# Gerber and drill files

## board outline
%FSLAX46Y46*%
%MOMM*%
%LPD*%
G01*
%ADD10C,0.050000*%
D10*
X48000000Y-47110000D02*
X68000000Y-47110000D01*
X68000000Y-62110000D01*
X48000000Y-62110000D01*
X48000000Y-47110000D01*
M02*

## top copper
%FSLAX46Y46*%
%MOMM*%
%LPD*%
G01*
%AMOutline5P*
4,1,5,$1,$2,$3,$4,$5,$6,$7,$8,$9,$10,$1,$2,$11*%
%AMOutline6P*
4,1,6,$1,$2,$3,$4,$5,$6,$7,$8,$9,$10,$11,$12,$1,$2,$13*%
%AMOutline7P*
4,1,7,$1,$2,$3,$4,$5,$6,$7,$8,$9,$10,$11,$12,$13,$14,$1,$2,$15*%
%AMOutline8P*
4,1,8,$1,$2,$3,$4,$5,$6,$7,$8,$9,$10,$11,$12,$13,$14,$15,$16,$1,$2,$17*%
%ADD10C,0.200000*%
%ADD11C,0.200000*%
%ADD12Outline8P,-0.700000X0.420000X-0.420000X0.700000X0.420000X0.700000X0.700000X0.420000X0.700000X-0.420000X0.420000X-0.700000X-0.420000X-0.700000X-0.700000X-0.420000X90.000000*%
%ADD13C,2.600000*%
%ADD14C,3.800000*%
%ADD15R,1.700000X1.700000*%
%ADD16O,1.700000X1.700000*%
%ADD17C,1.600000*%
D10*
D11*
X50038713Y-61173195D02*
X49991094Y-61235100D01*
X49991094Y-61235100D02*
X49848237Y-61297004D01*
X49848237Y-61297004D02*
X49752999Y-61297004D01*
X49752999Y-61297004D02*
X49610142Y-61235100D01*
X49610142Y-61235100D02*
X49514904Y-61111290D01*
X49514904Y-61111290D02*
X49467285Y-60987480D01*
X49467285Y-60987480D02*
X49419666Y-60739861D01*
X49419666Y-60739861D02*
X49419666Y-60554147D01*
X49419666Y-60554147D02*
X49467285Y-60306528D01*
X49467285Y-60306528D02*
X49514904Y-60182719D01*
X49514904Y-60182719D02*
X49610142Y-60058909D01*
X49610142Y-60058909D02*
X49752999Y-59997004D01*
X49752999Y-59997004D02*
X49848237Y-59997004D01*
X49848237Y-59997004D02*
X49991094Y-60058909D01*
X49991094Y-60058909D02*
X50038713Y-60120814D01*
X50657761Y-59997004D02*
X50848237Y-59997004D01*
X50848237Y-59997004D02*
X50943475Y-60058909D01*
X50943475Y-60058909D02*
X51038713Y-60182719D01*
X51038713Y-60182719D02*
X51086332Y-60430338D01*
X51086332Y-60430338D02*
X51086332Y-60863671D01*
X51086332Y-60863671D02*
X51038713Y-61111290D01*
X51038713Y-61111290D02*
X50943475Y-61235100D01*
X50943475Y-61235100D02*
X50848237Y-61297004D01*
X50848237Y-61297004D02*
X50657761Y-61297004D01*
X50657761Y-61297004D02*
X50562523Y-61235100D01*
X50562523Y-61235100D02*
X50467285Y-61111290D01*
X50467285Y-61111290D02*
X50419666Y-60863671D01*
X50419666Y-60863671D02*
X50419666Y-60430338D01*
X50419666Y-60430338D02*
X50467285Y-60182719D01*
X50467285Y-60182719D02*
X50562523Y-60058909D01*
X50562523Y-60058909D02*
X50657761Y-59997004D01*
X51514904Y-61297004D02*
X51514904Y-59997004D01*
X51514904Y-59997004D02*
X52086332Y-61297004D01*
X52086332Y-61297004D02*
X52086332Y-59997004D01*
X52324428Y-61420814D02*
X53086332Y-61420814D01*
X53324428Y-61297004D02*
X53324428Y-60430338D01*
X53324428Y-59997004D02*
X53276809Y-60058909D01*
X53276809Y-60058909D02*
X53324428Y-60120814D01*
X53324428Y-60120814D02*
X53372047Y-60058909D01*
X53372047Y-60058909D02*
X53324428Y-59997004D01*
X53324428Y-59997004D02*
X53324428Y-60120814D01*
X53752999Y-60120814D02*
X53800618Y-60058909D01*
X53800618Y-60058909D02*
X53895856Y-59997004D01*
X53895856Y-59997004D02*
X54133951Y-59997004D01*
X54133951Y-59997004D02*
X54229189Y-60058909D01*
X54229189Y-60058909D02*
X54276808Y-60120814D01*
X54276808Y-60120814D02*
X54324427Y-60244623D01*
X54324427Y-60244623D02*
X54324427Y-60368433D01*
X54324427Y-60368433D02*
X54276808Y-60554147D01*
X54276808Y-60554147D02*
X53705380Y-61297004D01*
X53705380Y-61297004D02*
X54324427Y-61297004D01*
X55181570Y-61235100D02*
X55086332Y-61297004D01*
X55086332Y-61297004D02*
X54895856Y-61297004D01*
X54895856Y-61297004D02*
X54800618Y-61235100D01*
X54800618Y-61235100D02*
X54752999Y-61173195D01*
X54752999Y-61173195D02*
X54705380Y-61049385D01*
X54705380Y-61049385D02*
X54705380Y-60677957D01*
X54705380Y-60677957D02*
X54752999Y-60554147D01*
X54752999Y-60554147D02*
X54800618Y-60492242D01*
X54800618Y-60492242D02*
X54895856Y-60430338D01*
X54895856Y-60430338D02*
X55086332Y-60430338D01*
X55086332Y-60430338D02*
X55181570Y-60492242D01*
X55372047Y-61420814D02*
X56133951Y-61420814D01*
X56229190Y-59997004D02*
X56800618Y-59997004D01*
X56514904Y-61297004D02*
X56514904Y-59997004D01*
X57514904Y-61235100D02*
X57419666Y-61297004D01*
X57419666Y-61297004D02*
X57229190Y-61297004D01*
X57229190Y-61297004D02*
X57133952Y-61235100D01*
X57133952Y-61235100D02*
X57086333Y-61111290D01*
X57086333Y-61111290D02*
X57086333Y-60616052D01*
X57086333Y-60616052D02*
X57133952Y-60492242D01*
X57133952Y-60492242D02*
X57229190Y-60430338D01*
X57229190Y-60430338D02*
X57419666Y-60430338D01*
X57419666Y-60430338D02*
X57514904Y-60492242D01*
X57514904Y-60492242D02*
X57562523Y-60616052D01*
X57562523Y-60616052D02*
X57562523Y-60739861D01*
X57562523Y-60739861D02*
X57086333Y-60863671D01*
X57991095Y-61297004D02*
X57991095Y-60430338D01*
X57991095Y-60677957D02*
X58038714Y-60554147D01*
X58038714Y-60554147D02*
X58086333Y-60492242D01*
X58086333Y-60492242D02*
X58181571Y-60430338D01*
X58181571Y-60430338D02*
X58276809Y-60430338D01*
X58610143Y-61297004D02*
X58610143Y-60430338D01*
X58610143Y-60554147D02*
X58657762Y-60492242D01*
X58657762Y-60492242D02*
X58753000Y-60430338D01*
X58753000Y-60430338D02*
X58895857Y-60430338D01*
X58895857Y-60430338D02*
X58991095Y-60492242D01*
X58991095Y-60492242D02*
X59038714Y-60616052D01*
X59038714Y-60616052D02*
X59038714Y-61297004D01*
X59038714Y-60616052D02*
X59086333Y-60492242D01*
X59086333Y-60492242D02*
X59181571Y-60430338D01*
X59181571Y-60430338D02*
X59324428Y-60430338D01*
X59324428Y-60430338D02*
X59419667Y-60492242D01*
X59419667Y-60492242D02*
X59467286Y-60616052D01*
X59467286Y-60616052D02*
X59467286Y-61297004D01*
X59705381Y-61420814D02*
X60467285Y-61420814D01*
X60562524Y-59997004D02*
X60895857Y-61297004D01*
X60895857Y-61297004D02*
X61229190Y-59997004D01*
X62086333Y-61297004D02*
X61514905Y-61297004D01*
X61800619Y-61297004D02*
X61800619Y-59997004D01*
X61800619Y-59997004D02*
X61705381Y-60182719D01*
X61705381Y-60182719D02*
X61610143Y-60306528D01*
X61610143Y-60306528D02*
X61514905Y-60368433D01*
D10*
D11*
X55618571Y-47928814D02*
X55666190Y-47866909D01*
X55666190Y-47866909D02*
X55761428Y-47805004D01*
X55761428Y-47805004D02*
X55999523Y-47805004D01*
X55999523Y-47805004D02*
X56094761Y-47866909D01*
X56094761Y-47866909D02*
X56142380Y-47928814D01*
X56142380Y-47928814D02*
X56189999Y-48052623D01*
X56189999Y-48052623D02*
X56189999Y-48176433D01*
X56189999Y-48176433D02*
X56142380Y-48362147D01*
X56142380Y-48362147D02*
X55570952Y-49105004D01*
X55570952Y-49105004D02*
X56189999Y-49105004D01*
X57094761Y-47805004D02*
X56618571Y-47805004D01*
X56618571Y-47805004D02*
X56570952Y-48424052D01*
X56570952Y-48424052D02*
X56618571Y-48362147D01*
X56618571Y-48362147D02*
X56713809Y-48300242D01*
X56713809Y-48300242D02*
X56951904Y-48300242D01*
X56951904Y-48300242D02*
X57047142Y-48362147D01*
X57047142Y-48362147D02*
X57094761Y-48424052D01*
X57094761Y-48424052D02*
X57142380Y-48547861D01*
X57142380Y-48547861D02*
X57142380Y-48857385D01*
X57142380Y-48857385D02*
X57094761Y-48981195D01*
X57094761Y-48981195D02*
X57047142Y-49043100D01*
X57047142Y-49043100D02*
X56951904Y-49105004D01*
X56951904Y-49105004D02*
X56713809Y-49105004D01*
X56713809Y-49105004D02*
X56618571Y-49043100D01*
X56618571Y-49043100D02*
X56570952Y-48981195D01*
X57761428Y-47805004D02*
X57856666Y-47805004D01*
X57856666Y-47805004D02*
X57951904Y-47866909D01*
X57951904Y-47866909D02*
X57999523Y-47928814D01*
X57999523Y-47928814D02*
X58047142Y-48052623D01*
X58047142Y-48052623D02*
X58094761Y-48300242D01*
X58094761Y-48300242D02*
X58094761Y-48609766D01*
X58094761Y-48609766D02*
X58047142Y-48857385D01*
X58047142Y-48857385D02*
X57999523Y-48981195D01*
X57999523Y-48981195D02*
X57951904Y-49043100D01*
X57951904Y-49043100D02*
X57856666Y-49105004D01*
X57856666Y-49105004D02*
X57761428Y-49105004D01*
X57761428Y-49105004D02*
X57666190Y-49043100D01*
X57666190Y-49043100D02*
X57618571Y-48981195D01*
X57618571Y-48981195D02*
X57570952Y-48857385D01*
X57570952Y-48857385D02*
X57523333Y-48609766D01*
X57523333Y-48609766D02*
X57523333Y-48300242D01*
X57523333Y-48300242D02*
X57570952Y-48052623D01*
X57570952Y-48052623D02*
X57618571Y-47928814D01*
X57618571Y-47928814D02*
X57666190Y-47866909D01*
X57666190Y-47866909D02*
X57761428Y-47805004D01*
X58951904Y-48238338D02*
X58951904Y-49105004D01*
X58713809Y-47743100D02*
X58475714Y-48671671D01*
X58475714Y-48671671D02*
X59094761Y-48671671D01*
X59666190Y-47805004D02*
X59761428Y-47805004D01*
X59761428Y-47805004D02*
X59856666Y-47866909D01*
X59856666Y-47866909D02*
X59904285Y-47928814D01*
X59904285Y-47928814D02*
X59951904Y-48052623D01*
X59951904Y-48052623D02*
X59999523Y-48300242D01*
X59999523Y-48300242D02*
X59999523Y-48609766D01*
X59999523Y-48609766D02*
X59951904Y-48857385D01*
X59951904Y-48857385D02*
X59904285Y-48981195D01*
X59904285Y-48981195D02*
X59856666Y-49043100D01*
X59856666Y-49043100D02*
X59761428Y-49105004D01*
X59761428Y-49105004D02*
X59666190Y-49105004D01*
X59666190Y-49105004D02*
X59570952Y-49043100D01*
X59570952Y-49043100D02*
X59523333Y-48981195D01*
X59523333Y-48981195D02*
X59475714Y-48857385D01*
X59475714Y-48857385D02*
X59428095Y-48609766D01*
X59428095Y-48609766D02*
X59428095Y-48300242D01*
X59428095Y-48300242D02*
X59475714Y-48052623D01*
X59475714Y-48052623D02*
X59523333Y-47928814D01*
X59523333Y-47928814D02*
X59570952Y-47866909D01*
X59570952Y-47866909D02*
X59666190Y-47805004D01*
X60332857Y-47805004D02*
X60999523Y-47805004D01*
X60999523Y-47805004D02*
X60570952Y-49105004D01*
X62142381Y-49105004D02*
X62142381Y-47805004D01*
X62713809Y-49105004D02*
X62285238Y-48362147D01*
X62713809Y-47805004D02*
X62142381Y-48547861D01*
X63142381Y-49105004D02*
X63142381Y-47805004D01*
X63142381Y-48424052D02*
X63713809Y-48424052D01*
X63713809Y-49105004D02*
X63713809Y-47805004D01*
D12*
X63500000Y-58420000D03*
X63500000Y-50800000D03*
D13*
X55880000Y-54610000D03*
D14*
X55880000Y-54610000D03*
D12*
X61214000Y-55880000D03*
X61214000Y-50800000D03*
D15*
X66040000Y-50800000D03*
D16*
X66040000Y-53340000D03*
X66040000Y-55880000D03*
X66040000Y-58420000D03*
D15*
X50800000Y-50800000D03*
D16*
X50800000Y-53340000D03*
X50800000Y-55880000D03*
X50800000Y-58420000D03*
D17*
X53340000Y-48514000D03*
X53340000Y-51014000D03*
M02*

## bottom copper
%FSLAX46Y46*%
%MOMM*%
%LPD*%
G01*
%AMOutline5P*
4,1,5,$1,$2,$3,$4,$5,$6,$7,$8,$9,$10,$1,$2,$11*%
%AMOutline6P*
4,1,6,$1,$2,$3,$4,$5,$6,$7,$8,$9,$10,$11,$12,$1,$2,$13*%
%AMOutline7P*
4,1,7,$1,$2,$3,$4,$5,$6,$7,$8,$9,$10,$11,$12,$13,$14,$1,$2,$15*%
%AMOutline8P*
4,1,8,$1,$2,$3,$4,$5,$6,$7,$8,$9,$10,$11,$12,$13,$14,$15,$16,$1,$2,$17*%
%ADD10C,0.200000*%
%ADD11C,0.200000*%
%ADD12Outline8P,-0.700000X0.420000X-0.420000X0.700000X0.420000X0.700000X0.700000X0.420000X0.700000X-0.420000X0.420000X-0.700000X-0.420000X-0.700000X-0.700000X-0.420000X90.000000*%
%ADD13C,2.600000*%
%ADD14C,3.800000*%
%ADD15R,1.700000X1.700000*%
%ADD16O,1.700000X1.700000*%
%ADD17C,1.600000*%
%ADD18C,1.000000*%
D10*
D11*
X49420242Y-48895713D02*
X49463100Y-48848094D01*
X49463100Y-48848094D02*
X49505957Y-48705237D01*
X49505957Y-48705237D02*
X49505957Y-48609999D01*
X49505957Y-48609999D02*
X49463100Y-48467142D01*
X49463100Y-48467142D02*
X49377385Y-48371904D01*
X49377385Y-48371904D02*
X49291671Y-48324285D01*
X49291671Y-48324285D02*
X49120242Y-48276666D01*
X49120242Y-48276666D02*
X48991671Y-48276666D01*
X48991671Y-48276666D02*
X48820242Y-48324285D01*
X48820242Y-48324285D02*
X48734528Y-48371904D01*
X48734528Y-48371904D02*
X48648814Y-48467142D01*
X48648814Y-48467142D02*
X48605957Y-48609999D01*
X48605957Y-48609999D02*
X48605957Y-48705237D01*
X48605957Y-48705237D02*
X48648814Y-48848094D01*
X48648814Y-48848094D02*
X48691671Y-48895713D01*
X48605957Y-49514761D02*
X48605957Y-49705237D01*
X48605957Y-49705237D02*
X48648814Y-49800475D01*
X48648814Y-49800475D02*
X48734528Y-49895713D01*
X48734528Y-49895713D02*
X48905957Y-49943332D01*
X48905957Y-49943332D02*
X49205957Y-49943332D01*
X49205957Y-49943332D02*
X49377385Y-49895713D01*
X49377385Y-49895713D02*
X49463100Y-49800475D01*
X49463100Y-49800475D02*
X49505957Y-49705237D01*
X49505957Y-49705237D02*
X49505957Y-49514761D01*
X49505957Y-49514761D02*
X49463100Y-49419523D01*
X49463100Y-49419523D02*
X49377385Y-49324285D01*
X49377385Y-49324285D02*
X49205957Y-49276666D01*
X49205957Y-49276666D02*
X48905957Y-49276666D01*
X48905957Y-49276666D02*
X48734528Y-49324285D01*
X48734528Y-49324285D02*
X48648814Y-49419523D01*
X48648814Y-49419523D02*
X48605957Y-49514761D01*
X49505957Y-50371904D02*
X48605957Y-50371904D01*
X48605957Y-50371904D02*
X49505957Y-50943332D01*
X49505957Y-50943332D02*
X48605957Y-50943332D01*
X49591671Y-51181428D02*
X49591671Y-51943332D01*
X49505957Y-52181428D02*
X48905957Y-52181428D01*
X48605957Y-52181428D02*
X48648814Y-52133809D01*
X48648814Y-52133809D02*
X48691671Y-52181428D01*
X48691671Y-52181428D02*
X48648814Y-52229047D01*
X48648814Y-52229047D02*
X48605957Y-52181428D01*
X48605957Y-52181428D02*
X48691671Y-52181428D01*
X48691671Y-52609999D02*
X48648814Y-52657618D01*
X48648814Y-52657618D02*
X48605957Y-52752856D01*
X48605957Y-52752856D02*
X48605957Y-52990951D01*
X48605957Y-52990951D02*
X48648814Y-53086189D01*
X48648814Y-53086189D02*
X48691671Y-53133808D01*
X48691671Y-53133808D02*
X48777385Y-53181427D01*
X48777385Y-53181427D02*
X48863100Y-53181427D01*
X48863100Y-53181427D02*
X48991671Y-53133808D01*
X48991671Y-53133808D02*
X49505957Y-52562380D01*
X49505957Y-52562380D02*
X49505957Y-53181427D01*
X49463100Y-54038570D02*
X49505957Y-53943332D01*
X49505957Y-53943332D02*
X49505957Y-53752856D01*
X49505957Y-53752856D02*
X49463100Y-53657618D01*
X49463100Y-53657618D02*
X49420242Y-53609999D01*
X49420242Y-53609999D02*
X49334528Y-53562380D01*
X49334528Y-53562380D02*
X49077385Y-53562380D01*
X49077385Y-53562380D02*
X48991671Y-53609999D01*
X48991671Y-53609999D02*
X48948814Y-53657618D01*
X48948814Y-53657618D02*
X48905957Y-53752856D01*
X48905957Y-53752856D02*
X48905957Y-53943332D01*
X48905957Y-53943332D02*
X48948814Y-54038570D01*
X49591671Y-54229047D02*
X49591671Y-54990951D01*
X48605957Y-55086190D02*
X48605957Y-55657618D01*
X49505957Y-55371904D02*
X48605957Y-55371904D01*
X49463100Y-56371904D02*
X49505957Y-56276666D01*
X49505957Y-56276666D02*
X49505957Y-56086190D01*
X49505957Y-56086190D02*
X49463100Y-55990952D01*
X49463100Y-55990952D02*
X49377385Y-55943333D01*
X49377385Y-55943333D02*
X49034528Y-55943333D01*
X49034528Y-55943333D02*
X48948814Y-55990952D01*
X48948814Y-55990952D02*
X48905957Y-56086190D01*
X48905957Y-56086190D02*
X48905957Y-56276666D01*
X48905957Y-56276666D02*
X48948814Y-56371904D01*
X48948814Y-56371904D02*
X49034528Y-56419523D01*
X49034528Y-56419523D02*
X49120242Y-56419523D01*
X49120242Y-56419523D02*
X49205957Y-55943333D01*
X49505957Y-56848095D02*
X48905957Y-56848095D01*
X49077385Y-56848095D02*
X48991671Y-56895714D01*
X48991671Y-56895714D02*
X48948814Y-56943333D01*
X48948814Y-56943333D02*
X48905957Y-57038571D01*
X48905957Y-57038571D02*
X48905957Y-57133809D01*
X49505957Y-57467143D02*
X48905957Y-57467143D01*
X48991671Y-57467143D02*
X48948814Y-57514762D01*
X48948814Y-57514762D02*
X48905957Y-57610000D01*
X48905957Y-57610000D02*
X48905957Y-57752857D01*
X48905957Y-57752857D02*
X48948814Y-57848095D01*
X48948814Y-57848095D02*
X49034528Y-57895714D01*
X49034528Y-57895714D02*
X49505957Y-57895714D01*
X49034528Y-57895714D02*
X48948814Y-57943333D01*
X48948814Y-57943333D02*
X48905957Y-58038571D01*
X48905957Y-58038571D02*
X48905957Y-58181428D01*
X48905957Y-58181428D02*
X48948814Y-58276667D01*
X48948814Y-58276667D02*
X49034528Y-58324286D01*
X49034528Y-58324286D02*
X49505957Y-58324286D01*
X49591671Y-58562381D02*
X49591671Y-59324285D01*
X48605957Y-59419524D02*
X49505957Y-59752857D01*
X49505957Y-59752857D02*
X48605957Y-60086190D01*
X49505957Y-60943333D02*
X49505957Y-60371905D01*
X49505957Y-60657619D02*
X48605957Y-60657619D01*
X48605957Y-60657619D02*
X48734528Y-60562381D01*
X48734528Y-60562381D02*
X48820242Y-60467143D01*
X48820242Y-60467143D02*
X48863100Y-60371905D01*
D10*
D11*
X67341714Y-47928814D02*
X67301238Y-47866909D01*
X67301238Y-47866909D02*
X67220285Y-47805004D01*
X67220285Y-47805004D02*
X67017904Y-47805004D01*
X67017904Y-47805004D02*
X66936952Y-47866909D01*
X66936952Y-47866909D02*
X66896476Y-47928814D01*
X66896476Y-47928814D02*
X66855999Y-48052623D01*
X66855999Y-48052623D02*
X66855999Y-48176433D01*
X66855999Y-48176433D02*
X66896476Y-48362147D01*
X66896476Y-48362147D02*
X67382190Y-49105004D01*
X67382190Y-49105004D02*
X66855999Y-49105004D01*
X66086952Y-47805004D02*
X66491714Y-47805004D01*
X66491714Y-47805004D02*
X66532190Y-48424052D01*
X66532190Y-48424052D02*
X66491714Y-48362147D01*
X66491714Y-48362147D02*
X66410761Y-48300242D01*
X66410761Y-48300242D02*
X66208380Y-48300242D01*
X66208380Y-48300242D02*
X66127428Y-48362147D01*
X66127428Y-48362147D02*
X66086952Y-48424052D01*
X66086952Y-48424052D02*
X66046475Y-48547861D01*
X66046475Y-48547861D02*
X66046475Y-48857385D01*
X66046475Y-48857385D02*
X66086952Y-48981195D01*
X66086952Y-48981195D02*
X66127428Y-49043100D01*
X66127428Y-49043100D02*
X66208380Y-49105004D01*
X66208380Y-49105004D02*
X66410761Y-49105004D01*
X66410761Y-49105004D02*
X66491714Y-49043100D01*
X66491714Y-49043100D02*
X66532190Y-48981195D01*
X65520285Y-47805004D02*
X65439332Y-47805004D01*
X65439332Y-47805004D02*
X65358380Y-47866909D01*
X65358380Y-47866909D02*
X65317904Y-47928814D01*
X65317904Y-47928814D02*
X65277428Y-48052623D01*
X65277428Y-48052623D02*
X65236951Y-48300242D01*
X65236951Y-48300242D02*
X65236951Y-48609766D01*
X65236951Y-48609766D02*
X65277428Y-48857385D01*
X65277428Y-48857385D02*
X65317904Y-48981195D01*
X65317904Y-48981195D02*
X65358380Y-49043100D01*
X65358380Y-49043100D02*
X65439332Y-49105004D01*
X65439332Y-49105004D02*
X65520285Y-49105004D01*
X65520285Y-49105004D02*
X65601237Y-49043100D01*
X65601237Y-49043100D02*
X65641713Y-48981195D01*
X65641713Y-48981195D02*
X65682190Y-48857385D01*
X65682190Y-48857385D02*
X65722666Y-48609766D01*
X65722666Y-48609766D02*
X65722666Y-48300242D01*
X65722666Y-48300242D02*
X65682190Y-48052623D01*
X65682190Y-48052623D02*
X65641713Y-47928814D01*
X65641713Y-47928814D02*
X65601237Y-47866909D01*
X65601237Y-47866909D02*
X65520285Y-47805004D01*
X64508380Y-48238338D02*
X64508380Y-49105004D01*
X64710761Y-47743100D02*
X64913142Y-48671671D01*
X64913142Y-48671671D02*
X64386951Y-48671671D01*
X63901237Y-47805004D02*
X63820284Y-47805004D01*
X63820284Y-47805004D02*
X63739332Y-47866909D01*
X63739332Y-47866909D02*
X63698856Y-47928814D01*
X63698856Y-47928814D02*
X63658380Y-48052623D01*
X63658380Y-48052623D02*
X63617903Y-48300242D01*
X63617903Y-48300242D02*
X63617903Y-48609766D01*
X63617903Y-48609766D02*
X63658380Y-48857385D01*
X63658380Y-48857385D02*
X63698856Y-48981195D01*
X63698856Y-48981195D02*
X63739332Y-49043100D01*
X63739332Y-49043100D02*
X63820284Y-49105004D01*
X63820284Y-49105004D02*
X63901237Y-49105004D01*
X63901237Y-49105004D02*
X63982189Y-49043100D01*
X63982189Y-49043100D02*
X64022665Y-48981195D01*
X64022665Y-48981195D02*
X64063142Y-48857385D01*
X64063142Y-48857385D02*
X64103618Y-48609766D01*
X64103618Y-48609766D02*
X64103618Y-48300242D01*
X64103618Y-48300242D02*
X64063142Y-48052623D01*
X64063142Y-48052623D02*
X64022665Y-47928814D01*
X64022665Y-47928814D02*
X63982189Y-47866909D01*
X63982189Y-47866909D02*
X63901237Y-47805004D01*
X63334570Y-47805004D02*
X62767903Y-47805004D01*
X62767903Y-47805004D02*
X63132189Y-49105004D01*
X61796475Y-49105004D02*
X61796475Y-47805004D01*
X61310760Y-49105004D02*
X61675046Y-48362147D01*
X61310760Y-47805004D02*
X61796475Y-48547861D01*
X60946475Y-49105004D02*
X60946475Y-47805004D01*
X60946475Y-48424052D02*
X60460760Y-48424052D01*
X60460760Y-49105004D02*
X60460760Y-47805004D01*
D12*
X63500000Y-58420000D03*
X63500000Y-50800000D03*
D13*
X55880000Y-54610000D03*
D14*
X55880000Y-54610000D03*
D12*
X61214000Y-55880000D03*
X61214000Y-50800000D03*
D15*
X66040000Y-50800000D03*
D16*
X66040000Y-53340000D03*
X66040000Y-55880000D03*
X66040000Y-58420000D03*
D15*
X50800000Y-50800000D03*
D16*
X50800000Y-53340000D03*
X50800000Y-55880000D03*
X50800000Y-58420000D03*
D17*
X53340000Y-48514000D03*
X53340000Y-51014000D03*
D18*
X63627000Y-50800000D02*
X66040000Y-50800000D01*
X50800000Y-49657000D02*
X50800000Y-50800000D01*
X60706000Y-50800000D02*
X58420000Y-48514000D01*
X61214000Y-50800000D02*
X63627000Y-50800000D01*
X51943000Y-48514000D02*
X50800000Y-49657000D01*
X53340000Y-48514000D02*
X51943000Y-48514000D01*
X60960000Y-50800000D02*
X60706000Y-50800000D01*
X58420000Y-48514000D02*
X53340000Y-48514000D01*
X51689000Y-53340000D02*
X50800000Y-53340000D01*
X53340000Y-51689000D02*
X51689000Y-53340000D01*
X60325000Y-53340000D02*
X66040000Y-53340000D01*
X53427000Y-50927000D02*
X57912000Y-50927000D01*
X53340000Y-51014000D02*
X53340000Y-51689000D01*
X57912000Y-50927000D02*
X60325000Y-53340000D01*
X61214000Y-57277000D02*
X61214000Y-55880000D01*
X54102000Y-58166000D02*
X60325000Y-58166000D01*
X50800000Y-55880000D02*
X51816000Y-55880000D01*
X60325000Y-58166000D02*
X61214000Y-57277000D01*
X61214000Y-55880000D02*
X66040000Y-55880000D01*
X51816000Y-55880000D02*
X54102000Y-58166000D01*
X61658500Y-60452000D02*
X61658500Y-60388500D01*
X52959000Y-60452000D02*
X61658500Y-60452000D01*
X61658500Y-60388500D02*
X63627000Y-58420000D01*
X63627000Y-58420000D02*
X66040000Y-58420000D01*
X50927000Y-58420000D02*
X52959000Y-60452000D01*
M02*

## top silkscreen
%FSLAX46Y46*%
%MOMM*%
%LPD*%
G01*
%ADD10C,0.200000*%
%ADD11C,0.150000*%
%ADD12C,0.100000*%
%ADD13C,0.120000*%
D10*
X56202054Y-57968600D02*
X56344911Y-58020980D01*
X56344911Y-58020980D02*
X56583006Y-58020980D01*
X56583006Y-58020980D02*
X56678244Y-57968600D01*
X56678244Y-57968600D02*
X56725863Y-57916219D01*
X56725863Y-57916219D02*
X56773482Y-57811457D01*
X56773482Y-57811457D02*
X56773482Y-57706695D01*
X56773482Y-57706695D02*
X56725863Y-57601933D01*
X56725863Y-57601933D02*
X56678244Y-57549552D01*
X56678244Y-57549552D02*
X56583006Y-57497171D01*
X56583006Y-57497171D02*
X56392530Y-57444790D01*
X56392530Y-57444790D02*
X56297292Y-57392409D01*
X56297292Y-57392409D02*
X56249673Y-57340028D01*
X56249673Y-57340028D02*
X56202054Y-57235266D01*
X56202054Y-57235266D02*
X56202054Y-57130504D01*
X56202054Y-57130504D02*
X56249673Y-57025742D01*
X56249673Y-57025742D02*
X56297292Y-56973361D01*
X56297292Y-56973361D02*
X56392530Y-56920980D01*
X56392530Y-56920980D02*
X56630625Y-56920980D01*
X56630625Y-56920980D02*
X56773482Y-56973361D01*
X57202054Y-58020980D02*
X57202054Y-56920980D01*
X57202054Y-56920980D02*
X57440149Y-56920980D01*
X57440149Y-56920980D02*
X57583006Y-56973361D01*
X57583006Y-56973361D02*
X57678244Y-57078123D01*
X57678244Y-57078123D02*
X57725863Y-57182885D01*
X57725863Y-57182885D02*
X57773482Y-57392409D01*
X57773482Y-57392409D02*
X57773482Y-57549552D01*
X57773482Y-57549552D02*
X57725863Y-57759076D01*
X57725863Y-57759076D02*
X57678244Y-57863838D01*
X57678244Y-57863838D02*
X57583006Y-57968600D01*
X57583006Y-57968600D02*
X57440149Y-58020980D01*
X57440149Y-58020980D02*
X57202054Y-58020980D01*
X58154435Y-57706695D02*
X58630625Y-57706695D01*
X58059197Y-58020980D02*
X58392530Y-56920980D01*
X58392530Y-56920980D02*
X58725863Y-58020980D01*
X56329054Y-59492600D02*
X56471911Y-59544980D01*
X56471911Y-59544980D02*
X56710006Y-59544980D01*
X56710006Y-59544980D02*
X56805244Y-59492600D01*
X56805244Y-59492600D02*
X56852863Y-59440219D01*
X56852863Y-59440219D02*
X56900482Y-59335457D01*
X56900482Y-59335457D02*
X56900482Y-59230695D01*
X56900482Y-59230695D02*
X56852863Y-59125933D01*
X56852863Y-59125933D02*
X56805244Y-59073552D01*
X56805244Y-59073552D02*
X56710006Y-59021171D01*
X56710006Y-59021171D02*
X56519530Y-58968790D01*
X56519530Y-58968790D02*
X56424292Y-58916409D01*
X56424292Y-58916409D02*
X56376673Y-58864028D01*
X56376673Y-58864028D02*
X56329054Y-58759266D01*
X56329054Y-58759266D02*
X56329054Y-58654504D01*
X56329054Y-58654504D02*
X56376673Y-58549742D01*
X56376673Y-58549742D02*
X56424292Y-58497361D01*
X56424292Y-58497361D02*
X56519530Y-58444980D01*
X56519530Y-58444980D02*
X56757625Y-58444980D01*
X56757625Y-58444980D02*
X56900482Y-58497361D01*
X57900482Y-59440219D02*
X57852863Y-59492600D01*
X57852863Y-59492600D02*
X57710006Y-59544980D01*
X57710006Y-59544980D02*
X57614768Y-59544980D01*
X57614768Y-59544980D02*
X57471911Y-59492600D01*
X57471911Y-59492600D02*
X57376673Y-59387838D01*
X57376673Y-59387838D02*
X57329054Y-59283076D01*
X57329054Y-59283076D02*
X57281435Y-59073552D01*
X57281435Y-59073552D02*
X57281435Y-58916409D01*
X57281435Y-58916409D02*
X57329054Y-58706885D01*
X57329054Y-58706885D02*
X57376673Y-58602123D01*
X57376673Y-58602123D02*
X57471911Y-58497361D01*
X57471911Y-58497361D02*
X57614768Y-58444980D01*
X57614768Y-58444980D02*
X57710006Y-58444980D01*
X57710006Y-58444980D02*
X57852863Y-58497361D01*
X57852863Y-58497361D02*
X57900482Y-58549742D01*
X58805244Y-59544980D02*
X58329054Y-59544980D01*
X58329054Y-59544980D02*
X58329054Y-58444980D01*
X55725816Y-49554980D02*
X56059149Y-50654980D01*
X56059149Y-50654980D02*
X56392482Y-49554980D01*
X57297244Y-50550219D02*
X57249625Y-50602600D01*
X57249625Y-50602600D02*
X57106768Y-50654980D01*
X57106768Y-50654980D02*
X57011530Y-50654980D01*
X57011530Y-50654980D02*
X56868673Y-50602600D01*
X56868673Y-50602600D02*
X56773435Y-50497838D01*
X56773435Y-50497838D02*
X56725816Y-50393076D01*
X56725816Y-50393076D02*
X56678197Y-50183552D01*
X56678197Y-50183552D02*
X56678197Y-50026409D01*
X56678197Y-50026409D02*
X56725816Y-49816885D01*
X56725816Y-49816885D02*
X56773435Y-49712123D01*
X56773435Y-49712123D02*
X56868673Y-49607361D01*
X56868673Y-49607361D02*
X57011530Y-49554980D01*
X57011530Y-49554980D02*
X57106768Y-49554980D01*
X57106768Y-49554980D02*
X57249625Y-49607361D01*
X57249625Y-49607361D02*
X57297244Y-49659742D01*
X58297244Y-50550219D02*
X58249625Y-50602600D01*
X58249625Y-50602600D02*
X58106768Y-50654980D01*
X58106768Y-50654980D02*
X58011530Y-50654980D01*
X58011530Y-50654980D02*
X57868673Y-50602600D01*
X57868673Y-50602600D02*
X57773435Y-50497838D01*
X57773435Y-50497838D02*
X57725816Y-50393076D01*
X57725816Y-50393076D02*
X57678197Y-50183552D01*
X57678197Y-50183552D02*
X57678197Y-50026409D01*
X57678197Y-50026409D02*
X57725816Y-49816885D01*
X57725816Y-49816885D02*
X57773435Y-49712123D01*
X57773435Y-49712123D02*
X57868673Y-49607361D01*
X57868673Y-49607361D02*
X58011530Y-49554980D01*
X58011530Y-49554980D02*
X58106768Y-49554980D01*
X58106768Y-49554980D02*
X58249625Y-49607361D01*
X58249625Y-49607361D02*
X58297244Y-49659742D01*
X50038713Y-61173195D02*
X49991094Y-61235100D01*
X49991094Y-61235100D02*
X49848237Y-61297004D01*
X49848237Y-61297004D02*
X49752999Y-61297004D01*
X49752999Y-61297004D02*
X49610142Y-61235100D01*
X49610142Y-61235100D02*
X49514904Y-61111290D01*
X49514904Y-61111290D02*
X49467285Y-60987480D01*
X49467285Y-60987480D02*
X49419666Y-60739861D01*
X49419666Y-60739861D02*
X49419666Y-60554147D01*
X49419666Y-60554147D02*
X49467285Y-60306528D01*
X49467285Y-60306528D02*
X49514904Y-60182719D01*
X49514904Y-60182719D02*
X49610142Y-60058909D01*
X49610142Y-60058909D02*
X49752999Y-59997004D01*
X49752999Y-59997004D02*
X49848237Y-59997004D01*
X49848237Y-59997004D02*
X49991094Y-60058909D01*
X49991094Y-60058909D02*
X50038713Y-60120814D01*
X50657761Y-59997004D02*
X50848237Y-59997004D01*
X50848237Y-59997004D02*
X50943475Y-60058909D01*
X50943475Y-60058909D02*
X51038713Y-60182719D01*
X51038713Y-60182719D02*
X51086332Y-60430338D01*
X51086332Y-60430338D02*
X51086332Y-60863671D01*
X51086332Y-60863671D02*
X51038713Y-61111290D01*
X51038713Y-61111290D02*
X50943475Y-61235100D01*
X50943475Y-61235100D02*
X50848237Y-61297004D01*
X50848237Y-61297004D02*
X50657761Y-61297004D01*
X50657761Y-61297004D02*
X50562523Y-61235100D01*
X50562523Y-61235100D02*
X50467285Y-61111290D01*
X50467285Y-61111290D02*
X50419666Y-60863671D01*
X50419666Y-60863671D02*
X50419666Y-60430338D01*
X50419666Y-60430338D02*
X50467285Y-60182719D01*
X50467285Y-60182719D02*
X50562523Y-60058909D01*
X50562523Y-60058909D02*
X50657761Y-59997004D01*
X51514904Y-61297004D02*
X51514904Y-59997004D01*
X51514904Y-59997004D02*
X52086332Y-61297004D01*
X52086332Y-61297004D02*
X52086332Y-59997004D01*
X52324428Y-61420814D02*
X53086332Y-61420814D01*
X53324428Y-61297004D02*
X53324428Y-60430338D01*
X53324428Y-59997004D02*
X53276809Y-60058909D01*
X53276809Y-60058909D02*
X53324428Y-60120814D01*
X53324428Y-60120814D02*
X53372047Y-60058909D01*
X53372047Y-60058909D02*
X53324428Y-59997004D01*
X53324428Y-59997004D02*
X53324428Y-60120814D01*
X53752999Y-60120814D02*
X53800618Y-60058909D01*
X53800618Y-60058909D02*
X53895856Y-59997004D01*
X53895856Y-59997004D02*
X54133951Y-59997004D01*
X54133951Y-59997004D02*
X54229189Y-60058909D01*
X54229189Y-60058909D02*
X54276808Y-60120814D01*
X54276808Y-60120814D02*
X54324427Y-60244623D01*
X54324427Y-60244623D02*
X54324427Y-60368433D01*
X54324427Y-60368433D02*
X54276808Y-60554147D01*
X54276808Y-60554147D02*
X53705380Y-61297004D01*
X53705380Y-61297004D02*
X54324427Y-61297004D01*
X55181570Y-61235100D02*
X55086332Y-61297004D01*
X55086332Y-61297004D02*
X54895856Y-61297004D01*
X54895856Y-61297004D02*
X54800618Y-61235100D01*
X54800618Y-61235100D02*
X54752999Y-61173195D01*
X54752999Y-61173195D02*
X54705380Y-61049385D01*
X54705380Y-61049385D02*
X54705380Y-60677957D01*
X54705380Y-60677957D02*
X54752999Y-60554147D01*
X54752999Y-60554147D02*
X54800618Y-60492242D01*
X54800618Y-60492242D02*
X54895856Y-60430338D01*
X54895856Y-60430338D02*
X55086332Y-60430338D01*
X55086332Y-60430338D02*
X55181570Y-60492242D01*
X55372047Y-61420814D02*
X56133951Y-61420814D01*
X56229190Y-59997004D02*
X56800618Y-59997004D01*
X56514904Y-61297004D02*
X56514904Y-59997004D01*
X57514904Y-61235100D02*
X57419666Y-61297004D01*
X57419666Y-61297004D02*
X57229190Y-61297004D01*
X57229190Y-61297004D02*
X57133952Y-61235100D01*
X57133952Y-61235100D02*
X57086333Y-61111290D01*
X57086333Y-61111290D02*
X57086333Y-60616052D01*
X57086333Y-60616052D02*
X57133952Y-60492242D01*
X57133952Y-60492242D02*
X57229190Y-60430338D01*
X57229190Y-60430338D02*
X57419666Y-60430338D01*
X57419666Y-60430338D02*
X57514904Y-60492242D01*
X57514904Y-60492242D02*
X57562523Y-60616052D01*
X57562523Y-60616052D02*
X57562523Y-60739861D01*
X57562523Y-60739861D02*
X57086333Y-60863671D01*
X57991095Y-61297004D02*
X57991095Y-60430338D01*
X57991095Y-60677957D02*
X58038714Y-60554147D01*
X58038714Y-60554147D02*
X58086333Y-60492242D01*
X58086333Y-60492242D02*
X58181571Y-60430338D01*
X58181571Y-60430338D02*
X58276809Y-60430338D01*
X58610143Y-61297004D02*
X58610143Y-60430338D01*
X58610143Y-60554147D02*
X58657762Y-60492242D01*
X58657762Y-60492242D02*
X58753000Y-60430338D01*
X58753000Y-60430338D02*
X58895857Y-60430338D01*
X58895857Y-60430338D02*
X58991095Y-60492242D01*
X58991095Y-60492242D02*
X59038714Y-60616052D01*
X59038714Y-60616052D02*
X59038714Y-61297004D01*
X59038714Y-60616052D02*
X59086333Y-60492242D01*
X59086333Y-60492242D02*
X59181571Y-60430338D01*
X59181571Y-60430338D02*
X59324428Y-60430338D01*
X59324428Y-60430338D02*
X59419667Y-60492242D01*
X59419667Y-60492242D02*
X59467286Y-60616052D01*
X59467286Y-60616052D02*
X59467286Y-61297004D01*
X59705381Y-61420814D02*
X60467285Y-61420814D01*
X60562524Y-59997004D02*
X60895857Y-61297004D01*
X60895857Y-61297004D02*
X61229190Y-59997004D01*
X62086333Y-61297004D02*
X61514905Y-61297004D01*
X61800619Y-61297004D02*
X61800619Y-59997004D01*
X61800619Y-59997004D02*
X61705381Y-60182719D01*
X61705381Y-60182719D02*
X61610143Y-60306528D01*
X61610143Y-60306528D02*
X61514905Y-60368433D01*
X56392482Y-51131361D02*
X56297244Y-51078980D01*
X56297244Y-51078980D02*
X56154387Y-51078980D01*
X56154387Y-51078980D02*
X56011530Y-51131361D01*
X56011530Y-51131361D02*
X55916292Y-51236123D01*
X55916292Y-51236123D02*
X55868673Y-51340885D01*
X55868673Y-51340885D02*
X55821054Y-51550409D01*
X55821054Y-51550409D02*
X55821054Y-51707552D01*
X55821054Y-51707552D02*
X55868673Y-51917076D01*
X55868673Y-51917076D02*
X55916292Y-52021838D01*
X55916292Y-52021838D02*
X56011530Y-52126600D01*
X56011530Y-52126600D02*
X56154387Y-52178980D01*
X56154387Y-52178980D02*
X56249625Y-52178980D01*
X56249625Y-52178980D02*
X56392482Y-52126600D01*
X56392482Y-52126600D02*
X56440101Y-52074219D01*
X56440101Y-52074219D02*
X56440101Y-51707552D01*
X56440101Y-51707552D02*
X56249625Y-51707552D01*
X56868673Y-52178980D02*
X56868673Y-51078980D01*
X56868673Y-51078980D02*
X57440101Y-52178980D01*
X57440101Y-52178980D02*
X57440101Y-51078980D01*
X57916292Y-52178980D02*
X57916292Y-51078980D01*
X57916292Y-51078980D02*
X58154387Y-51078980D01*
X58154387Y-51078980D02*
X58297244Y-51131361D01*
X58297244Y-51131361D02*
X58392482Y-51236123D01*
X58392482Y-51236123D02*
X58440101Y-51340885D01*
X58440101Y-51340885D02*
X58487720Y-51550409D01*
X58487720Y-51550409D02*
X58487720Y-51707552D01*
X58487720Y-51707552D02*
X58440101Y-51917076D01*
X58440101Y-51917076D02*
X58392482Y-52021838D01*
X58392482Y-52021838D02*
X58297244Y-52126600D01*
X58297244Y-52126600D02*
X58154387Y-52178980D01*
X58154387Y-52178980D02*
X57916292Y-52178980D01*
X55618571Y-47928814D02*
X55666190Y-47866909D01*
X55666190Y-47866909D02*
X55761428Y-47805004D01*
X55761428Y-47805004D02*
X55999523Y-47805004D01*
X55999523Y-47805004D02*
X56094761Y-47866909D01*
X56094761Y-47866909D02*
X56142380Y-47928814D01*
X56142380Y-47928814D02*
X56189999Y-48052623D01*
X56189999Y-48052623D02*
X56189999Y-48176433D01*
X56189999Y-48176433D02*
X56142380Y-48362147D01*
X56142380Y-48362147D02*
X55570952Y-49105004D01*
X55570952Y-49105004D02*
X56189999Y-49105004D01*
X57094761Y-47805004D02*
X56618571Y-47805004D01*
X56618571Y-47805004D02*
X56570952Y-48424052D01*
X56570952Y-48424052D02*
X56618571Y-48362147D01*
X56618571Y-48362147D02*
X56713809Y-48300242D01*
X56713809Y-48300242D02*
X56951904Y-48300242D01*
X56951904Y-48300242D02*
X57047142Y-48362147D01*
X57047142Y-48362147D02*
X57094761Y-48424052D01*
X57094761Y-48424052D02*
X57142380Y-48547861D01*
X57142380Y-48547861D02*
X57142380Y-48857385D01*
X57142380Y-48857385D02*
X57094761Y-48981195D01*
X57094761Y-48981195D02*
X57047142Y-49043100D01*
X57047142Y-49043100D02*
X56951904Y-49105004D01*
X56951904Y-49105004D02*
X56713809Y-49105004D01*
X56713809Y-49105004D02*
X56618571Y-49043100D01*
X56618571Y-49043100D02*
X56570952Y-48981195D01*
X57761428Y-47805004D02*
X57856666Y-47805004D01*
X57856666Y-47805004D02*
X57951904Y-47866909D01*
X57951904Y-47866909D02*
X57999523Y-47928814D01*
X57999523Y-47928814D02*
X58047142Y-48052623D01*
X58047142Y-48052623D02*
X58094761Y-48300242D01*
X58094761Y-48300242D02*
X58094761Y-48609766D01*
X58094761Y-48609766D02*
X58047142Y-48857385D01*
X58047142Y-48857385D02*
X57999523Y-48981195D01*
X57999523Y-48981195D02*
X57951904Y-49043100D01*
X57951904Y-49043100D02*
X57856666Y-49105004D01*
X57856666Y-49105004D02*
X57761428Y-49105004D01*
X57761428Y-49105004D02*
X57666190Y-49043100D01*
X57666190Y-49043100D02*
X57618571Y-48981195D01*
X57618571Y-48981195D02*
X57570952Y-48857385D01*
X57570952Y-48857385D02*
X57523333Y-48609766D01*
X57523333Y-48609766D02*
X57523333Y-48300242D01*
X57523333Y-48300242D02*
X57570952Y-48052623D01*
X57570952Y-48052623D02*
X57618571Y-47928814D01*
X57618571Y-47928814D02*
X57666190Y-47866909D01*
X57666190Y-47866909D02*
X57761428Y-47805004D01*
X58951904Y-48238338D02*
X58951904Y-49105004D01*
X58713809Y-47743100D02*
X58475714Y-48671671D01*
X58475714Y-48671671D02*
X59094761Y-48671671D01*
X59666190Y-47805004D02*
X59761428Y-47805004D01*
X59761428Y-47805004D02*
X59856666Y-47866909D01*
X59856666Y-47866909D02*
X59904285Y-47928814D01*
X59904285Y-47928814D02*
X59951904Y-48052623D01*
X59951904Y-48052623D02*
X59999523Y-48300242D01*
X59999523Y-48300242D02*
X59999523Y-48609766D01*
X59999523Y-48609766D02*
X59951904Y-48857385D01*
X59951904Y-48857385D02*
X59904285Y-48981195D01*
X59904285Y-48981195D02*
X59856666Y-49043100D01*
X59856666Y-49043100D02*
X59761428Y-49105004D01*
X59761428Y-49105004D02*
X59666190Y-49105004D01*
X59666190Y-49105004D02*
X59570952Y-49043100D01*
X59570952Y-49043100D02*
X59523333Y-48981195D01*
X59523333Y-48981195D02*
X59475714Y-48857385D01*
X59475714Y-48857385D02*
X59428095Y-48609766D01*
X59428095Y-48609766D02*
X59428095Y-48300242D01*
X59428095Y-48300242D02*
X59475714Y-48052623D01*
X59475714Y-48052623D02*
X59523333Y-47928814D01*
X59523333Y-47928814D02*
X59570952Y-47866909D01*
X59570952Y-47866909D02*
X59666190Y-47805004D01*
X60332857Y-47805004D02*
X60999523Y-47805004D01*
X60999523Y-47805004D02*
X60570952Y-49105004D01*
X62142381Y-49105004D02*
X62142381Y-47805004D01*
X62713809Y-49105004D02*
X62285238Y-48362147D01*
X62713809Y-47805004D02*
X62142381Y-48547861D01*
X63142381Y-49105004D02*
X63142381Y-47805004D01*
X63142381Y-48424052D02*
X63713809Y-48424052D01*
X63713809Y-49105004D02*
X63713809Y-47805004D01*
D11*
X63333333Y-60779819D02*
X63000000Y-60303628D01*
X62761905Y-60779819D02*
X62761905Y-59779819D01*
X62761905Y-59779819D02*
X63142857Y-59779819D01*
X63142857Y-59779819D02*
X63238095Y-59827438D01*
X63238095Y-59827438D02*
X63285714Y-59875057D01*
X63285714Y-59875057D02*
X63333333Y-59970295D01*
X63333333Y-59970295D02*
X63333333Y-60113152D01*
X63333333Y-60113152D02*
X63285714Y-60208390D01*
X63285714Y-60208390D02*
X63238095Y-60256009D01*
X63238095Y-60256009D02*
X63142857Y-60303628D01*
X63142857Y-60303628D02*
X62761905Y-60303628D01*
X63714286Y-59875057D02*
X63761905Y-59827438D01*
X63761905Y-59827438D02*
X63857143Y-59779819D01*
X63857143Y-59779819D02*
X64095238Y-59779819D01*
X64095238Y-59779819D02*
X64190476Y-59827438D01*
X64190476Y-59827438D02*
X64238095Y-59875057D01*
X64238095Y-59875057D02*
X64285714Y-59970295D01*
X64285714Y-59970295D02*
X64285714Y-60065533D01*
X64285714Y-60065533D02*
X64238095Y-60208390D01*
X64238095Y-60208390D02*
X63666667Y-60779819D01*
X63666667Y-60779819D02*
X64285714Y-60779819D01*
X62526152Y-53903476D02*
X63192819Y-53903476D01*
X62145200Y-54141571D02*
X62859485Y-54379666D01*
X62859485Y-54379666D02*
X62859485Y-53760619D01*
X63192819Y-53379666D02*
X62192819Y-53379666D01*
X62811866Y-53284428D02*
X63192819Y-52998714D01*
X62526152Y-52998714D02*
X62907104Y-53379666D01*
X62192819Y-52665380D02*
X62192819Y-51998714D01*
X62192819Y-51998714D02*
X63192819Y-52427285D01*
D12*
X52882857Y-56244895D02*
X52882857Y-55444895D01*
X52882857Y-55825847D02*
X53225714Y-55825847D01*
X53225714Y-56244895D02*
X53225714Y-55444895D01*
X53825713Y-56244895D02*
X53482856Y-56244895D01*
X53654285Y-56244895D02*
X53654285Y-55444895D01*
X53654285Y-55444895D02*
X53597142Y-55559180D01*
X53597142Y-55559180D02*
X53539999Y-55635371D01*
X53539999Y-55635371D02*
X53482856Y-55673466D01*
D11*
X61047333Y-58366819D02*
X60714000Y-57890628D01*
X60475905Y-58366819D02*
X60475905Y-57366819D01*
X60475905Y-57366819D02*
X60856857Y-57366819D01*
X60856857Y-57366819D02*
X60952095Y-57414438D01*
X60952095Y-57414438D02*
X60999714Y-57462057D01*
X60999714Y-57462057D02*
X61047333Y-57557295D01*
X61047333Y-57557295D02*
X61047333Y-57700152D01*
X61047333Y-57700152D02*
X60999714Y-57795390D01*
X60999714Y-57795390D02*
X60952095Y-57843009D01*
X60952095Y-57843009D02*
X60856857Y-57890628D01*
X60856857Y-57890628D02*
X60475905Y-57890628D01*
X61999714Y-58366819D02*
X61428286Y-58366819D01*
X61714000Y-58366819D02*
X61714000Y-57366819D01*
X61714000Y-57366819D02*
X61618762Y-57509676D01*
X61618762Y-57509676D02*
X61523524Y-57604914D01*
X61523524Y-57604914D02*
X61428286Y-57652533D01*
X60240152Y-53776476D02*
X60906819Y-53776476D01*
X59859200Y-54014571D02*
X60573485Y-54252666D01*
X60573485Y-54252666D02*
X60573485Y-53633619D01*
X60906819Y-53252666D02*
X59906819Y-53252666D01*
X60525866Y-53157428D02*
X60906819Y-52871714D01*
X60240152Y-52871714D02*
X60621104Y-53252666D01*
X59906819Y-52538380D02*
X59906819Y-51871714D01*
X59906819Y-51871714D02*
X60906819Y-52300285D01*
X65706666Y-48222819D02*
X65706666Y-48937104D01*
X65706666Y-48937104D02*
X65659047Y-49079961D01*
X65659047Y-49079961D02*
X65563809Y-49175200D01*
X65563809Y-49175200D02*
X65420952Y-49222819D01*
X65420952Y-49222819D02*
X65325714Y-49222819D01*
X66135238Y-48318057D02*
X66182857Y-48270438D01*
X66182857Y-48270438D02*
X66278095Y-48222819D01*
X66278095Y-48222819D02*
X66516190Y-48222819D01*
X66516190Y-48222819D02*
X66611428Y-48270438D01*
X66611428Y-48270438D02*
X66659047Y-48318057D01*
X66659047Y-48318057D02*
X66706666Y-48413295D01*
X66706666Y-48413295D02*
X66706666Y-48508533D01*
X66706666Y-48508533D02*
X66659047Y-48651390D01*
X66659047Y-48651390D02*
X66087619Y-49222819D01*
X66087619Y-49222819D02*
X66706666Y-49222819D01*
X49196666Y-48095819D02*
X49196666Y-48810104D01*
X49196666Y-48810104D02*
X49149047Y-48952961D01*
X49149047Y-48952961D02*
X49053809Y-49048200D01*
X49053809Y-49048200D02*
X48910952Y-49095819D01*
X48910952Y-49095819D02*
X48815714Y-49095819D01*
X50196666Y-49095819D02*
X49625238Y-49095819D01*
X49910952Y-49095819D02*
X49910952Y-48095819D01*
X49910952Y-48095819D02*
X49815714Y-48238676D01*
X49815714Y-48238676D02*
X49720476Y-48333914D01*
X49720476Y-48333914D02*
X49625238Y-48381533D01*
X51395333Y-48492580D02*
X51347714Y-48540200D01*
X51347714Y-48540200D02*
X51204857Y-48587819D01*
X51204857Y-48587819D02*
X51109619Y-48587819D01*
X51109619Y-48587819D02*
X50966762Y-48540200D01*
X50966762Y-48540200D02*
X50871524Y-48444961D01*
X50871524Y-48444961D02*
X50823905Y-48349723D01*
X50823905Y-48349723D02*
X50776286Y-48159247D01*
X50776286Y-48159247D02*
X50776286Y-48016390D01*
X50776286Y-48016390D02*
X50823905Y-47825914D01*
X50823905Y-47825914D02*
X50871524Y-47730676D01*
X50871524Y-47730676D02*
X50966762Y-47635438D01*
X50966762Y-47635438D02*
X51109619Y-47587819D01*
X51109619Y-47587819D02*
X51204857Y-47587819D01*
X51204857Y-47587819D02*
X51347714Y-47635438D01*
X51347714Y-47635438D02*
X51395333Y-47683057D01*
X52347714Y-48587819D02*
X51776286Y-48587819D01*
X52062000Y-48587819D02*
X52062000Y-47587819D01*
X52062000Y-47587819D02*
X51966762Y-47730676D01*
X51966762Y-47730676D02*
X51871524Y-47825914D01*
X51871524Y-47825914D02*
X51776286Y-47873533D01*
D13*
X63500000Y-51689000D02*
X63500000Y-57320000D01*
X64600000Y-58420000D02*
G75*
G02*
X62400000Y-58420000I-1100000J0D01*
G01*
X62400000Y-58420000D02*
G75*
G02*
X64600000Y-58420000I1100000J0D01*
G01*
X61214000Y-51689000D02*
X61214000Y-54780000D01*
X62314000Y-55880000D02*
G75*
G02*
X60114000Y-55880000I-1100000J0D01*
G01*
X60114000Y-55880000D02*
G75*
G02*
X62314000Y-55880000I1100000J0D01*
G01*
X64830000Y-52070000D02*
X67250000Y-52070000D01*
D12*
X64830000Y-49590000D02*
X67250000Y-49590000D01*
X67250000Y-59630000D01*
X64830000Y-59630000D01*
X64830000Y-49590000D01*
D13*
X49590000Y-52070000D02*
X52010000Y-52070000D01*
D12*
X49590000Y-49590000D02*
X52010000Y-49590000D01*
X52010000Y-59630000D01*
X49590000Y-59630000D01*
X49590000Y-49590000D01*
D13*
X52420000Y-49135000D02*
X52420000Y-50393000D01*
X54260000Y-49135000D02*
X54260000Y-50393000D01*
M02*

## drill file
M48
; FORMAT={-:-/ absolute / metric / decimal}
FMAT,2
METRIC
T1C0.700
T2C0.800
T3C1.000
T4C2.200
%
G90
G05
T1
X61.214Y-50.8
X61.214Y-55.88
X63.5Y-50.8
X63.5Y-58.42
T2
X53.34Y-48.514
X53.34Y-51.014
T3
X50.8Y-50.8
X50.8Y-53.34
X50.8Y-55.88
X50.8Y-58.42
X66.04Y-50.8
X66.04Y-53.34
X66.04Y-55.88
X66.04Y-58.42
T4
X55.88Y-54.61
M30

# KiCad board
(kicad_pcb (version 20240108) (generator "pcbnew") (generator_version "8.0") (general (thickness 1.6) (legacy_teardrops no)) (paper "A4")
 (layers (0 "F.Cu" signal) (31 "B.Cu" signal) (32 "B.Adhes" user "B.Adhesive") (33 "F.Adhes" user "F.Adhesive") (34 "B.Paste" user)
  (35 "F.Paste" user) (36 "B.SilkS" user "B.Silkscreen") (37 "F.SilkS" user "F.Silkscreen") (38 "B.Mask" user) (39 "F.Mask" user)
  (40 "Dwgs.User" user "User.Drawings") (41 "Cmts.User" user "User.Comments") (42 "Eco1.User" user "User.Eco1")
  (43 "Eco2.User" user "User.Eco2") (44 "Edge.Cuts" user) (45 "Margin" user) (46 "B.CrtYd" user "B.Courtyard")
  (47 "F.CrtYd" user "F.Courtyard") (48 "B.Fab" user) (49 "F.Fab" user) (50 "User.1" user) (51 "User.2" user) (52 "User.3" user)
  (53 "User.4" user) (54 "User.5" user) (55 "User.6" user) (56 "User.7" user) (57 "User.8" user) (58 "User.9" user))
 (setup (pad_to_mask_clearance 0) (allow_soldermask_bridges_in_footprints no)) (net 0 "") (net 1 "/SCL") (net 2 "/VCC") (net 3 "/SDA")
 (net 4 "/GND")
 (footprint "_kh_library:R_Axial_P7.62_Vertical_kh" (layer "F.Cu") (at 63.5 58.42 90)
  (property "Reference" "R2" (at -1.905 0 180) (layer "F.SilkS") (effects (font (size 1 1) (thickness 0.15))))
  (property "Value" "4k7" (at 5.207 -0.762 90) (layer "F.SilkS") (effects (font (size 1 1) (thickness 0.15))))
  (fp_line (start 6.731 0) (end 1.1 0) (stroke (width 0.12) (type solid)) (layer "F.SilkS"))
  (fp_circle (center 0 0) (end 1.1 0) (stroke (width 0.12) (type solid)) (fill none) (layer "F.SilkS"))
  (pad "1" thru_hole roundrect (at 0 0 90) (size 1.4 1.4) (drill 0.7) (layers "*.Cu" "*.Mask") (remove_unused_layers no)
   (roundrect_rratio 0) (chamfer_ratio 0.2) (chamfer top_left top_right bottom_left bottom_right) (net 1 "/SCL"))
  (pad "2" thru_hole roundrect (at 7.62 0 90) (size 1.4 1.4) (drill 0.7) (layers "*.Cu" "*.Mask") (remove_unused_layers no)
   (roundrect_rratio 0) (chamfer_ratio 0.2) (chamfer top_left top_right bottom_left bottom_right) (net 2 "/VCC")))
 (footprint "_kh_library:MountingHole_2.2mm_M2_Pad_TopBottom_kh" (layer "F.Cu") (at 55.88 54.61)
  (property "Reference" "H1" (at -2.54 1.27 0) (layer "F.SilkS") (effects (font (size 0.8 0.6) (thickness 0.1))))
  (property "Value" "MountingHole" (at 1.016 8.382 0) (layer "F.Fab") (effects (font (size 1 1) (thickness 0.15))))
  (pad "1" thru_hole circle (at 0 0) (size 2.6 2.6) (drill 2.2) (layers "*.Cu" "*.Mask") (remove_unused_layers no))
  (pad "1" connect circle (at 0 0) (size 3.8 3.8) (layers "F.Cu" "F.Mask"))
  (pad "1" connect circle (at 0 0) (size 3.8 3.8) (layers "B.Cu" "B.Mask")))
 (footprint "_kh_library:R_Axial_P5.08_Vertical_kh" (layer "F.Cu") (at 61.214 55.88 90)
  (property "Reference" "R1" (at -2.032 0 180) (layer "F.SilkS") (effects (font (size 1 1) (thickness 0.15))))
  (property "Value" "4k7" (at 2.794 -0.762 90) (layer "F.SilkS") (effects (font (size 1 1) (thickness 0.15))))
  (fp_line (start 4.191 0) (end 1.1 0) (stroke (width 0.12) (type solid)) (layer "F.SilkS"))
  (fp_circle (center 0 0) (end 1.1 0) (stroke (width 0.12) (type solid)) (fill none) (layer "F.SilkS"))
  (pad "1" thru_hole roundrect (at 0 0 90) (size 1.4 1.4) (drill 0.7) (layers "*.Cu" "*.Mask") (remove_unused_layers no)
   (roundrect_rratio 0) (chamfer_ratio 0.2) (chamfer top_left top_right bottom_left bottom_right) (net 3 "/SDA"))
  (pad "2" thru_hole roundrect (at 5.08 0 90) (size 1.4 1.4) (drill 0.7) (layers "*.Cu" "*.Mask") (remove_unused_layers no)
   (roundrect_rratio 0) (chamfer_ratio 0.2) (chamfer top_left top_right bottom_left bottom_right) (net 2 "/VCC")))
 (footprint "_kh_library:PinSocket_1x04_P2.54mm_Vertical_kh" (layer "F.Cu") (at 66.04 50.8)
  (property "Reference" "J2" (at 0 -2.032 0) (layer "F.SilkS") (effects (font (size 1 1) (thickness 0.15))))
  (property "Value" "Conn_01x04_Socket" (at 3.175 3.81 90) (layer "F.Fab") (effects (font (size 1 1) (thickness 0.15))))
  (fp_line (start -1.21 1.27) (end 1.21 1.27) (stroke (width 0.12) (type solid)) (layer "F.SilkS"))
  (fp_rect (start -1.21 -1.21) (end 1.21 8.83) (stroke (width 0.1) (type default)) (fill none) (layer "F.SilkS"))
  (pad "1" thru_hole rect (at 0 0) (size 1.7 1.7) (drill 1) (layers "*.Cu" "*.Mask") (remove_unused_layers no) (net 2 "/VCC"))
  (pad "2" thru_hole oval (at 0 2.54) (size 1.7 1.7) (drill 1) (layers "*.Cu" "*.Mask") (remove_unused_layers no) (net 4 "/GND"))
  (pad "3" thru_hole oval (at 0 5.08) (size 1.7 1.7) (drill 1) (layers "*.Cu" "*.Mask") (remove_unused_layers no) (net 3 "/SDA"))
  (pad "4" thru_hole oval (at 0 7.62) (size 1.7 1.7) (drill 1) (layers "*.Cu" "*.Mask") (remove_unused_layers no) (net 1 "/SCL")))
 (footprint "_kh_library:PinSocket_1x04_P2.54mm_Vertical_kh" (layer "F.Cu") (at 50.8 50.8)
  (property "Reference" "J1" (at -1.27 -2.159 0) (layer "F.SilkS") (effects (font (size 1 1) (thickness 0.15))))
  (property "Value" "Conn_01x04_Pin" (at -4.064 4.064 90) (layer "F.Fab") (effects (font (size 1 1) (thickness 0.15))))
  (fp_line (start -1.21 1.27) (end 1.21 1.27) (stroke (width 0.12) (type solid)) (layer "F.SilkS"))
  (fp_rect (start -1.21 -1.21) (end 1.21 8.83) (stroke (width 0.1) (type default)) (fill none) (layer "F.SilkS"))
  (pad "1" thru_hole rect (at 0 0) (size 1.7 1.7) (drill 1) (layers "*.Cu" "*.Mask") (remove_unused_layers no) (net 2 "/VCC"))
  (pad "2" thru_hole oval (at 0 2.54) (size 1.7 1.7) (drill 1) (layers "*.Cu" "*.Mask") (remove_unused_layers no) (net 4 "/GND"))
  (pad "3" thru_hole oval (at 0 5.08) (size 1.7 1.7) (drill 1) (layers "*.Cu" "*.Mask") (remove_unused_layers no) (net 3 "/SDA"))
  (pad "4" thru_hole oval (at 0 7.62) (size 1.7 1.7) (drill 1) (layers "*.Cu" "*.Mask") (remove_unused_layers no) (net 1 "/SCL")))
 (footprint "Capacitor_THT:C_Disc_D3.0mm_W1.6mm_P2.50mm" (layer "F.Cu") (at 53.34 48.514 -90)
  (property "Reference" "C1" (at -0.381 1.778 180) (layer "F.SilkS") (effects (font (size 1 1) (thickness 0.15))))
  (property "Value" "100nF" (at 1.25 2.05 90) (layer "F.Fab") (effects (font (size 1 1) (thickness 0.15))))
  (fp_line (start 0.621 0.92) (end 1.879 0.92) (stroke (width 0.12) (type solid)) (layer "F.SilkS"))
  (fp_line (start 0.621 -0.92) (end 1.879 -0.92) (stroke (width 0.12) (type solid)) (layer "F.SilkS"))
  (pad "1" thru_hole circle (at 0 0 270) (size 1.6 1.6) (drill 0.8) (layers "*.Cu" "*.Mask") (remove_unused_layers no) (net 2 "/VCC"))
  (pad "2" thru_hole circle (at 2.5 0 270) (size 1.6 1.6) (drill 0.8) (layers "*.Cu" "*.Mask") (remove_unused_layers no) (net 4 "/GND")))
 (gr_rect (start 48 47.11) (end 68 62.11) (stroke (width 0.05) (type default)) (fill none) (layer "Edge.Cuts"))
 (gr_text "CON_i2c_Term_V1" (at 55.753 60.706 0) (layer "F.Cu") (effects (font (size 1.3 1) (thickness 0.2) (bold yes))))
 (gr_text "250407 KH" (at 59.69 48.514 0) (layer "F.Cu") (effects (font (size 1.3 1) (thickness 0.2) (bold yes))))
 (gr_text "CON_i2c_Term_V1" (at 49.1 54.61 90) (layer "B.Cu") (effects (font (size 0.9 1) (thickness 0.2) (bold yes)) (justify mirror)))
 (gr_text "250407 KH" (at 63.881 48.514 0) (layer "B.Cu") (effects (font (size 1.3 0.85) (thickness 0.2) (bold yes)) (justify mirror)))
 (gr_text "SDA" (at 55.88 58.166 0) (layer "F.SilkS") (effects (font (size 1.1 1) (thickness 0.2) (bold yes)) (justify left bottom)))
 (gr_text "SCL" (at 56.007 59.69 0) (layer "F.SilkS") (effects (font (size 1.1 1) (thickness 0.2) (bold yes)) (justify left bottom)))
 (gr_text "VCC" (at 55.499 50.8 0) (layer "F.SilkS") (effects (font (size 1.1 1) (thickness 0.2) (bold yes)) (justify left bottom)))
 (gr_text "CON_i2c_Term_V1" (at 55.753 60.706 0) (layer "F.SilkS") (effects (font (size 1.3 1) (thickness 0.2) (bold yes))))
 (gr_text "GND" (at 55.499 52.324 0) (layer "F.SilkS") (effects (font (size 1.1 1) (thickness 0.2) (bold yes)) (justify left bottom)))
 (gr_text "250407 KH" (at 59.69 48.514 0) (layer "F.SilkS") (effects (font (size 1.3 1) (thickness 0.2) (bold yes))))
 (segment (start 63.627 50.8) (end 66.04 50.8) (width 1) (layer "B.Cu") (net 2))
 (segment (start 50.8 49.657) (end 50.8 50.8) (width 1) (layer "B.Cu") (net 2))
 (segment (start 60.706 50.8) (end 58.42 48.514) (width 1) (layer "B.Cu") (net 2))
 (segment (start 61.214 50.8) (end 63.627 50.8) (width 1) (layer "B.Cu") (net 2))
 (segment (start 51.943 48.514) (end 50.8 49.657) (width 1) (layer "B.Cu") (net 2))
 (segment (start 53.34 48.514) (end 51.943 48.514) (width 1) (layer "B.Cu") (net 2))
 (segment (start 60.96 50.8) (end 60.706 50.8) (width 1) (layer "B.Cu") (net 2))
 (segment (start 58.42 48.514) (end 53.34 48.514) (width 1) (layer "B.Cu") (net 2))
 (segment (start 51.689 53.34) (end 50.8 53.34) (width 1) (layer "B.Cu") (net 4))
 (segment (start 53.34 51.689) (end 51.689 53.34) (width 1) (layer "B.Cu") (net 4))
 (segment (start 60.325 53.34) (end 66.04 53.34) (width 1) (layer "B.Cu") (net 4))
 (segment (start 53.427 50.927) (end 57.912 50.927) (width 1) (layer "B.Cu") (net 4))
 (segment (start 53.34 51.014) (end 53.34 51.689) (width 1) (layer "B.Cu") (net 4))
 (segment (start 57.912 50.927) (end 60.325 53.34) (width 1) (layer "B.Cu") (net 4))
 (segment (start 61.214 57.277) (end 61.214 55.88) (width 1) (layer "B.Cu") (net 3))
 (segment (start 54.102 58.166) (end 60.325 58.166) (width 1) (layer "B.Cu") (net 3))
 (segment (start 50.8 55.88) (end 51.816 55.88) (width 1) (layer "B.Cu") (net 3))
 (segment (start 60.325 58.166) (end 61.214 57.277) (width 1) (layer "B.Cu") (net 3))
 (segment (start 61.214 55.88) (end 66.04 55.88) (width 1) (layer "B.Cu") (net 3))
 (segment (start 51.816 55.88) (end 54.102 58.166) (width 1) (layer "B.Cu") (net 3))
 (segment (start 61.6585 60.452) (end 61.6585 60.3885) (width 1) (layer "B.Cu") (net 1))
 (segment (start 52.959 60.452) (end 61.6585 60.452) (width 1) (layer "B.Cu") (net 1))
 (segment (start 61.6585 60.3885) (end 63.627 58.42) (width 1) (layer "B.Cu") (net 1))
 (segment (start 63.627 58.42) (end 66.04 58.42) (width 1) (layer "B.Cu") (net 1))
 (segment (start 50.927 58.42) (end 52.959 60.452) (width 1) (layer "B.Cu") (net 1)))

